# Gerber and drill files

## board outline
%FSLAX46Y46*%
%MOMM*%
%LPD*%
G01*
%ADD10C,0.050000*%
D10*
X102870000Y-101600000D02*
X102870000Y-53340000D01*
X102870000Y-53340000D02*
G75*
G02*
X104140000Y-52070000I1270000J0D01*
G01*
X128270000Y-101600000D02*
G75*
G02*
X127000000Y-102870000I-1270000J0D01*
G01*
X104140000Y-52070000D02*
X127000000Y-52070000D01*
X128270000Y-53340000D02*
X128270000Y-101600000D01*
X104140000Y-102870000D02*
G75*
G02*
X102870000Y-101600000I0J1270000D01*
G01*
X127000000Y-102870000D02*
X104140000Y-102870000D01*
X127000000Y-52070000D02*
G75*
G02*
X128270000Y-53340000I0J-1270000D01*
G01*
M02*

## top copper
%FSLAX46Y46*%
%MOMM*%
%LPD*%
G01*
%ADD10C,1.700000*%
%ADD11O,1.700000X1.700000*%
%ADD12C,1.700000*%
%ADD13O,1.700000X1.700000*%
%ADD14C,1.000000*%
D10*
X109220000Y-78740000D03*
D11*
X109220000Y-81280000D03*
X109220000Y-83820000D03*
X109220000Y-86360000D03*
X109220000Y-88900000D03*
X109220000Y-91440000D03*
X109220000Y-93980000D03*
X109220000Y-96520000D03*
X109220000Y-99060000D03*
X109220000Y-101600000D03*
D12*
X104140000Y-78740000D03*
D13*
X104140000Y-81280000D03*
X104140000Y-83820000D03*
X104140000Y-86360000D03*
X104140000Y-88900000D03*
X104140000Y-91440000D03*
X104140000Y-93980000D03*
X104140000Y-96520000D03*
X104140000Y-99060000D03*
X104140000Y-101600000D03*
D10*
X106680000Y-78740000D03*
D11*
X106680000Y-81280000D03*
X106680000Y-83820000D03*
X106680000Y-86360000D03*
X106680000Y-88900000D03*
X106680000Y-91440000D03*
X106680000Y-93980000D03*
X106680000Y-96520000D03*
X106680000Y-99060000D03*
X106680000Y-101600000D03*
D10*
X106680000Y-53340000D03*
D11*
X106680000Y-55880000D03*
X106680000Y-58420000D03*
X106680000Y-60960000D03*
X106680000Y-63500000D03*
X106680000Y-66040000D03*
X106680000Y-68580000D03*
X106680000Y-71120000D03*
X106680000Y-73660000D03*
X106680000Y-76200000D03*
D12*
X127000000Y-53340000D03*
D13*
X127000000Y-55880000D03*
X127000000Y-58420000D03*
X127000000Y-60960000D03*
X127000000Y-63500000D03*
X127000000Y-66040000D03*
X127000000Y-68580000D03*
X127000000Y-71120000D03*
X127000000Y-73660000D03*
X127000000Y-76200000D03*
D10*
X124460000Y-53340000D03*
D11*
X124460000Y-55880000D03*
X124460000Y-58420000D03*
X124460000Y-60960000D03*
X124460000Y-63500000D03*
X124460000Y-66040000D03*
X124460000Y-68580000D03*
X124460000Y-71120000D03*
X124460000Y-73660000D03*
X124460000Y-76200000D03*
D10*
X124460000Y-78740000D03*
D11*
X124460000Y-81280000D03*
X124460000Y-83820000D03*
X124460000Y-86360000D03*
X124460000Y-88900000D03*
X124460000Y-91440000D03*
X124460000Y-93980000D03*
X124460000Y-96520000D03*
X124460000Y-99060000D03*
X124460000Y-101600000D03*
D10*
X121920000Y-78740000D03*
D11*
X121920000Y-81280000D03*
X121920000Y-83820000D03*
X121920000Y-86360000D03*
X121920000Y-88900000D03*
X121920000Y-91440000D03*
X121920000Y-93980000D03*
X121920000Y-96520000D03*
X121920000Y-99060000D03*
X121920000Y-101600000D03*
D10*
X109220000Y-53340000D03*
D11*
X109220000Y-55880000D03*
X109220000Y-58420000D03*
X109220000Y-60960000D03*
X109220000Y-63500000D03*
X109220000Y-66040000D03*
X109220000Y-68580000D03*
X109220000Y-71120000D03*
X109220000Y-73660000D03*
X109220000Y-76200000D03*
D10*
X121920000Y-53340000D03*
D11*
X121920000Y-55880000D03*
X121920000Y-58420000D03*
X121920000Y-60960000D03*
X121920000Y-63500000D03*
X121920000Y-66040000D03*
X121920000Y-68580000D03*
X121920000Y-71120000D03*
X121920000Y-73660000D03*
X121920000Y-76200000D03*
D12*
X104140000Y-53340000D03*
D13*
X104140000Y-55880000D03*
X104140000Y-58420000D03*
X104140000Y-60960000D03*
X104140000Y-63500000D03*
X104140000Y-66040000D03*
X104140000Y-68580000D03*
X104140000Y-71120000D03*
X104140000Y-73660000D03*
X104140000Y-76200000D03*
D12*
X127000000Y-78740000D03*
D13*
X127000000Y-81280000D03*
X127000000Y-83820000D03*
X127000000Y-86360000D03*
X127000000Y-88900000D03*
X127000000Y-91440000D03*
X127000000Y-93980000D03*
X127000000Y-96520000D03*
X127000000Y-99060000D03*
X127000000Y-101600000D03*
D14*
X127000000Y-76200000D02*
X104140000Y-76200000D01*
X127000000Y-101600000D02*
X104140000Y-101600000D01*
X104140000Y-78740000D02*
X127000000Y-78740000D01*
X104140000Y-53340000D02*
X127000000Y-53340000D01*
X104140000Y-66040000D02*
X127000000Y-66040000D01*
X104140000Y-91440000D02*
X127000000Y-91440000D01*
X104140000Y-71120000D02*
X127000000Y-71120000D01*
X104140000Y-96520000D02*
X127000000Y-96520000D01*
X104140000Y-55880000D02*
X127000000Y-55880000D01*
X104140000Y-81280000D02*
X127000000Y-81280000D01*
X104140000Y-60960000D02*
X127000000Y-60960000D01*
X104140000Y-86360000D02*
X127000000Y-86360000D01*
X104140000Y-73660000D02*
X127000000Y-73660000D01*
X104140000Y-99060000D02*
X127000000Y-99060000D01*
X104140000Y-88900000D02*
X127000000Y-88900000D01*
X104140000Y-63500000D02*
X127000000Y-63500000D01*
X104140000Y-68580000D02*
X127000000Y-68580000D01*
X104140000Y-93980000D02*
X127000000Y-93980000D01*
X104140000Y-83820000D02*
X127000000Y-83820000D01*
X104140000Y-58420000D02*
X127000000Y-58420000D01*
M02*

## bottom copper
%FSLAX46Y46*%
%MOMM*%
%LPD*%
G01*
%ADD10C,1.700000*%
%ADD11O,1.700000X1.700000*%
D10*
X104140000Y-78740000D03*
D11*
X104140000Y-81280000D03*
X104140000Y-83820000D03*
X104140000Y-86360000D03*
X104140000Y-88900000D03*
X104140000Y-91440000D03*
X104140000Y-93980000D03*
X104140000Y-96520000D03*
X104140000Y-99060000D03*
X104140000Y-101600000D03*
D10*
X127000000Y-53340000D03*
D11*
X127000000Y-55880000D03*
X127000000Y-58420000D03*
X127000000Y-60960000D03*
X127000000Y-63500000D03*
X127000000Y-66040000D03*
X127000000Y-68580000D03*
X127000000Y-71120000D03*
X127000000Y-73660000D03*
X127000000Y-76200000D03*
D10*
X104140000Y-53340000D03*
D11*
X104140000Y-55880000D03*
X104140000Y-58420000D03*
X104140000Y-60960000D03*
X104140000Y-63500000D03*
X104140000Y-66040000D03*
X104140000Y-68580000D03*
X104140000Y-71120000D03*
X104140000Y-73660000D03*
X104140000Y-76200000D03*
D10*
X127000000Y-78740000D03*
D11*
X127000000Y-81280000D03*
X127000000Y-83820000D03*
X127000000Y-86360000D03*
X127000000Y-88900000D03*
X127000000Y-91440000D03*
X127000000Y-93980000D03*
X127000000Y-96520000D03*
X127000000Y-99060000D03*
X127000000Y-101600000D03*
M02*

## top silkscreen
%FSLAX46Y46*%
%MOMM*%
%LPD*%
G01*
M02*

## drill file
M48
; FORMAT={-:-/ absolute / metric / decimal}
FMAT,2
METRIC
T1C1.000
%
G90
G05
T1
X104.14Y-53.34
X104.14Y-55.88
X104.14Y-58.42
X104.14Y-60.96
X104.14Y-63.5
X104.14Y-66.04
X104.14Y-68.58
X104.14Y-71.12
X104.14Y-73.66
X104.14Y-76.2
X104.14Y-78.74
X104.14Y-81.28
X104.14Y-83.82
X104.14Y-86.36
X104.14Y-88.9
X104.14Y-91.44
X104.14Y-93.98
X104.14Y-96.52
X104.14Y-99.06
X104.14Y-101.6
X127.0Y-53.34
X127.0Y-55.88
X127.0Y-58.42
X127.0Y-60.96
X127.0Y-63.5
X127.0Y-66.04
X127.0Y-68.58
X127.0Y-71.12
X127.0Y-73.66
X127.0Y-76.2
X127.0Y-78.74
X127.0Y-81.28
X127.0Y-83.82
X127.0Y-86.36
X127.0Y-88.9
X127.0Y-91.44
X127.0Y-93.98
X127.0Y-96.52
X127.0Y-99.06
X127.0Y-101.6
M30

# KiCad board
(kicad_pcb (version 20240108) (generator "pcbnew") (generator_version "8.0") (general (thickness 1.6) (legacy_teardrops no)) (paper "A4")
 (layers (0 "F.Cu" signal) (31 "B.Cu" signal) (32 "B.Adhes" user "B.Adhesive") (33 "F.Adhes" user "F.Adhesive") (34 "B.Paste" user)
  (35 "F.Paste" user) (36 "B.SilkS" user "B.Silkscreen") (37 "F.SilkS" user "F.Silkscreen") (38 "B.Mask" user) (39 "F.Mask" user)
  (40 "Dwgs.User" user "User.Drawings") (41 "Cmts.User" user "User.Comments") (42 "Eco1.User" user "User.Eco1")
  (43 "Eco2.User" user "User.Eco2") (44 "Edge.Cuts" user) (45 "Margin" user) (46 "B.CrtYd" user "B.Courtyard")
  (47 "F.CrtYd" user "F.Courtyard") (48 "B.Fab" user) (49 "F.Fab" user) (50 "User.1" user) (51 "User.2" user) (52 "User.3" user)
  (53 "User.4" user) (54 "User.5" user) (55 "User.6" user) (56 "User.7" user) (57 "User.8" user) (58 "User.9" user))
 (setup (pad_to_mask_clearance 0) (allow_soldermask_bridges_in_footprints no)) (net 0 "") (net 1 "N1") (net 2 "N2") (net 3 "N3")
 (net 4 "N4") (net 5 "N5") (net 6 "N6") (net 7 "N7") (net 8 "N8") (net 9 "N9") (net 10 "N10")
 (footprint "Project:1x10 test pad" (layer "F.Cu") (at 109.22 90.065)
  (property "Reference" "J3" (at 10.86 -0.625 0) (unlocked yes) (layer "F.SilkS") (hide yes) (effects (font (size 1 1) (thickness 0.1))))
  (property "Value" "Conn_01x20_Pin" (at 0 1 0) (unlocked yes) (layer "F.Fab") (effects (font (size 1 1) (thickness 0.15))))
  (pad "1" smd circle (at 0 -11.325) (size 1.7 1.7) (layers "F.Cu" "F.Paste" "F.Mask") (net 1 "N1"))
  (pad "2" smd oval (at 0 -8.785) (size 1.7 1.7) (layers "F.Cu" "F.Paste" "F.Mask") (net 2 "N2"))
  (pad "3" smd oval (at 0 -6.245) (size 1.7 1.7) (layers "F.Cu" "F.Paste" "F.Mask") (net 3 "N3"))
  (pad "4" smd oval (at 0 -3.705) (size 1.7 1.7) (layers "F.Cu" "F.Paste" "F.Mask") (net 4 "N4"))
  (pad "5" smd oval (at 0 -1.165) (size 1.7 1.7) (layers "F.Cu" "F.Paste" "F.Mask") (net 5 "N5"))
  (pad "6" smd oval (at 0 1.375) (size 1.7 1.7) (layers "F.Cu" "F.Paste" "F.Mask") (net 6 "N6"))
  (pad "7" smd oval (at 0 3.915) (size 1.7 1.7) (layers "F.Cu" "F.Paste" "F.Mask") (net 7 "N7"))
  (pad "8" smd oval (at 0 6.455) (size 1.7 1.7) (layers "F.Cu" "F.Paste" "F.Mask") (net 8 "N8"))
  (pad "9" smd oval (at 0 8.995) (size 1.7 1.7) (layers "F.Cu" "F.Paste" "F.Mask") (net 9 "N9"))
  (pad "10" smd oval (at 0 11.535) (size 1.7 1.7) (layers "F.Cu" "F.Paste" "F.Mask") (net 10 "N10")))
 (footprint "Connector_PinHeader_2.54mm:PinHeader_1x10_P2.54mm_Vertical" (layer "F.Cu") (at 104.14 78.74)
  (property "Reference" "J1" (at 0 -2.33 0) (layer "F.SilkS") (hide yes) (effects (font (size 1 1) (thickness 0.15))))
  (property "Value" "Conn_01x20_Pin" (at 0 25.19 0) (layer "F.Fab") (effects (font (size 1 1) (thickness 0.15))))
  (pad "1" thru_hole circle (at 0 0) (size 1.7 1.7) (drill 1) (layers "*.Cu" "*.Mask") (remove_unused_layers no) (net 1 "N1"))
  (pad "2" thru_hole oval (at 0 2.54) (size 1.7 1.7) (drill 1) (layers "*.Cu" "*.Mask") (remove_unused_layers no) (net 2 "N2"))
  (pad "3" thru_hole oval (at 0 5.08) (size 1.7 1.7) (drill 1) (layers "*.Cu" "*.Mask") (remove_unused_layers no) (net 3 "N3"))
  (pad "4" thru_hole oval (at 0 7.62) (size 1.7 1.7) (drill 1) (layers "*.Cu" "*.Mask") (remove_unused_layers no) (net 4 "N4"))
  (pad "5" thru_hole oval (at 0 10.16) (size 1.7 1.7) (drill 1) (layers "*.Cu" "*.Mask") (remove_unused_layers no) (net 5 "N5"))
  (pad "6" thru_hole oval (at 0 12.7) (size 1.7 1.7) (drill 1) (layers "*.Cu" "*.Mask") (remove_unused_layers no) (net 6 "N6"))
  (pad "7" thru_hole oval (at 0 15.24) (size 1.7 1.7) (drill 1) (layers "*.Cu" "*.Mask") (remove_unused_layers no) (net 7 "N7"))
  (pad "8" thru_hole oval (at 0 17.78) (size 1.7 1.7) (drill 1) (layers "*.Cu" "*.Mask") (remove_unused_layers no) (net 8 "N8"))
  (pad "9" thru_hole oval (at 0 20.32) (size 1.7 1.7) (drill 1) (layers "*.Cu" "*.Mask") (remove_unused_layers no) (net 9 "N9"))
  (pad "10" thru_hole oval (at 0 22.86) (size 1.7 1.7) (drill 1) (layers "*.Cu" "*.Mask") (remove_unused_layers no) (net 10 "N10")))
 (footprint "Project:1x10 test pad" (layer "F.Cu") (at 106.68 90.065)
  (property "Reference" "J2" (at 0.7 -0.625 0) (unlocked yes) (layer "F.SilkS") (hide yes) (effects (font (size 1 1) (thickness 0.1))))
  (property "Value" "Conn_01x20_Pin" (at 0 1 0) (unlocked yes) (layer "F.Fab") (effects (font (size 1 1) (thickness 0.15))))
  (pad "1" smd circle (at 0 -11.325) (size 1.7 1.7) (layers "F.Cu" "F.Paste" "F.Mask") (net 1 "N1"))
  (pad "2" smd oval (at 0 -8.785) (size 1.7 1.7) (layers "F.Cu" "F.Paste" "F.Mask") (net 2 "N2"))
  (pad "3" smd oval (at 0 -6.245) (size 1.7 1.7) (layers "F.Cu" "F.Paste" "F.Mask") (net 3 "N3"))
  (pad "4" smd oval (at 0 -3.705) (size 1.7 1.7) (layers "F.Cu" "F.Paste" "F.Mask") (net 4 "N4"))
  (pad "5" smd oval (at 0 -1.165) (size 1.7 1.7) (layers "F.Cu" "F.Paste" "F.Mask") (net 5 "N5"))
  (pad "6" smd oval (at 0 1.375) (size 1.7 1.7) (layers "F.Cu" "F.Paste" "F.Mask") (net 6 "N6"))
  (pad "7" smd oval (at 0 3.915) (size 1.7 1.7) (layers "F.Cu" "F.Paste" "F.Mask") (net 7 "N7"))
  (pad "8" smd oval (at 0 6.455) (size 1.7 1.7) (layers "F.Cu" "F.Paste" "F.Mask") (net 8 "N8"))
  (pad "9" smd oval (at 0 8.995) (size 1.7 1.7) (layers "F.Cu" "F.Paste" "F.Mask") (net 9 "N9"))
  (pad "10" smd oval (at 0 11.535) (size 1.7 1.7) (layers "F.Cu" "F.Paste" "F.Mask") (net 10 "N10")))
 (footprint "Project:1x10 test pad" (layer "F.Cu") (at 106.68 64.665)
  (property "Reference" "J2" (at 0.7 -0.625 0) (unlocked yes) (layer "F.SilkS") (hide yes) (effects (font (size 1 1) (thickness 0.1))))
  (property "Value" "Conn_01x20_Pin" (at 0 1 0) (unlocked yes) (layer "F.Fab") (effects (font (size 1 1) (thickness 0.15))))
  (pad "1" smd circle (at 0 -11.325) (size 1.7 1.7) (layers "F.Cu" "F.Paste" "F.Mask") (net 1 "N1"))
  (pad "2" smd oval (at 0 -8.785) (size 1.7 1.7) (layers "F.Cu" "F.Paste" "F.Mask") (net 2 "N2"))
  (pad "3" smd oval (at 0 -6.245) (size 1.7 1.7) (layers "F.Cu" "F.Paste" "F.Mask") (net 3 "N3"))
  (pad "4" smd oval (at 0 -3.705) (size 1.7 1.7) (layers "F.Cu" "F.Paste" "F.Mask") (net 4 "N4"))
  (pad "5" smd oval (at 0 -1.165) (size 1.7 1.7) (layers "F.Cu" "F.Paste" "F.Mask") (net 5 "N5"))
  (pad "6" smd oval (at 0 1.375) (size 1.7 1.7) (layers "F.Cu" "F.Paste" "F.Mask") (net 6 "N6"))
  (pad "7" smd oval (at 0 3.915) (size 1.7 1.7) (layers "F.Cu" "F.Paste" "F.Mask") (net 7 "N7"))
  (pad "8" smd oval (at 0 6.455) (size 1.7 1.7) (layers "F.Cu" "F.Paste" "F.Mask") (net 8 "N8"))
  (pad "9" smd oval (at 0 8.995) (size 1.7 1.7) (layers "F.Cu" "F.Paste" "F.Mask") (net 9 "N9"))
  (pad "10" smd oval (at 0 11.535) (size 1.7 1.7) (layers "F.Cu" "F.Paste" "F.Mask") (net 10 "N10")))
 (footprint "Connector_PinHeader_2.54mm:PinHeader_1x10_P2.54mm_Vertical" (layer "F.Cu") (at 127 53.34)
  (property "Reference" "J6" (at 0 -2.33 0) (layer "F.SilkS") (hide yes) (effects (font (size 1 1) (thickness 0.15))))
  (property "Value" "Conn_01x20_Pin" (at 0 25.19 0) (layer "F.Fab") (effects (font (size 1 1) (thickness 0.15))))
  (pad "1" thru_hole circle (at 0 0) (size 1.7 1.7) (drill 1) (layers "*.Cu" "*.Mask") (remove_unused_layers no) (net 1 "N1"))
  (pad "2" thru_hole oval (at 0 2.54) (size 1.7 1.7) (drill 1) (layers "*.Cu" "*.Mask") (remove_unused_layers no) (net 2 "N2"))
  (pad "3" thru_hole oval (at 0 5.08) (size 1.7 1.7) (drill 1) (layers "*.Cu" "*.Mask") (remove_unused_layers no) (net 3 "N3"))
  (pad "4" thru_hole oval (at 0 7.62) (size 1.7 1.7) (drill 1) (layers "*.Cu" "*.Mask") (remove_unused_layers no) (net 4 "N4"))
  (pad "5" thru_hole oval (at 0 10.16) (size 1.7 1.7) (drill 1) (layers "*.Cu" "*.Mask") (remove_unused_layers no) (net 5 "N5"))
  (pad "6" thru_hole oval (at 0 12.7) (size 1.7 1.7) (drill 1) (layers "*.Cu" "*.Mask") (remove_unused_layers no) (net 6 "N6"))
  (pad "7" thru_hole oval (at 0 15.24) (size 1.7 1.7) (drill 1) (layers "*.Cu" "*.Mask") (remove_unused_layers no) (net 7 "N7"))
  (pad "8" thru_hole oval (at 0 17.78) (size 1.7 1.7) (drill 1) (layers "*.Cu" "*.Mask") (remove_unused_layers no) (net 8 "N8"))
  (pad "9" thru_hole oval (at 0 20.32) (size 1.7 1.7) (drill 1) (layers "*.Cu" "*.Mask") (remove_unused_layers no) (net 9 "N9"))
  (pad "10" thru_hole oval (at 0 22.86) (size 1.7 1.7) (drill 1) (layers "*.Cu" "*.Mask") (remove_unused_layers no) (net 10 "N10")))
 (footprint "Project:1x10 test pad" (layer "F.Cu") (at 124.46 64.665)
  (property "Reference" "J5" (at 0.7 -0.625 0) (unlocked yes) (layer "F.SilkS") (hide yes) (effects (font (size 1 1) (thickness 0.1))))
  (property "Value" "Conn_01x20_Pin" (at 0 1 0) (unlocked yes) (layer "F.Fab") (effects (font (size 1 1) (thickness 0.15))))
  (pad "1" smd circle (at 0 -11.325) (size 1.7 1.7) (layers "F.Cu" "F.Paste" "F.Mask") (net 1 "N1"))
  (pad "2" smd oval (at 0 -8.785) (size 1.7 1.7) (layers "F.Cu" "F.Paste" "F.Mask") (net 2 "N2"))
  (pad "3" smd oval (at 0 -6.245) (size 1.7 1.7) (layers "F.Cu" "F.Paste" "F.Mask") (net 3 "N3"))
  (pad "4" smd oval (at 0 -3.705) (size 1.7 1.7) (layers "F.Cu" "F.Paste" "F.Mask") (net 4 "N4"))
  (pad "5" smd oval (at 0 -1.165) (size 1.7 1.7) (layers "F.Cu" "F.Paste" "F.Mask") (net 5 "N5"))
  (pad "6" smd oval (at 0 1.375) (size 1.7 1.7) (layers "F.Cu" "F.Paste" "F.Mask") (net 6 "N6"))
  (pad "7" smd oval (at 0 3.915) (size 1.7 1.7) (layers "F.Cu" "F.Paste" "F.Mask") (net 7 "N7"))
  (pad "8" smd oval (at 0 6.455) (size 1.7 1.7) (layers "F.Cu" "F.Paste" "F.Mask") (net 8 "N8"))
  (pad "9" smd oval (at 0 8.995) (size 1.7 1.7) (layers "F.Cu" "F.Paste" "F.Mask") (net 9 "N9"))
  (pad "10" smd oval (at 0 11.535) (size 1.7 1.7) (layers "F.Cu" "F.Paste" "F.Mask") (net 10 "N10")))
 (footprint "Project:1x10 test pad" (layer "F.Cu") (at 124.46 90.065)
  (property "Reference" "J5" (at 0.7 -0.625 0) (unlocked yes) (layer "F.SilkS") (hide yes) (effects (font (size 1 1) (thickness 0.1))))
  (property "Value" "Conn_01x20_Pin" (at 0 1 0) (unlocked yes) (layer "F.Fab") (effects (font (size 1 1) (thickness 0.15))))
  (pad "1" smd circle (at 0 -11.325) (size 1.7 1.7) (layers "F.Cu" "F.Paste" "F.Mask") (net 1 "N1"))
  (pad "2" smd oval (at 0 -8.785) (size 1.7 1.7) (layers "F.Cu" "F.Paste" "F.Mask") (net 2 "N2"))
  (pad "3" smd oval (at 0 -6.245) (size 1.7 1.7) (layers "F.Cu" "F.Paste" "F.Mask") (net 3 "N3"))
  (pad "4" smd oval (at 0 -3.705) (size 1.7 1.7) (layers "F.Cu" "F.Paste" "F.Mask") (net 4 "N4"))
  (pad "5" smd oval (at 0 -1.165) (size 1.7 1.7) (layers "F.Cu" "F.Paste" "F.Mask") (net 5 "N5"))
  (pad "6" smd oval (at 0 1.375) (size 1.7 1.7) (layers "F.Cu" "F.Paste" "F.Mask") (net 6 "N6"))
  (pad "7" smd oval (at 0 3.915) (size 1.7 1.7) (layers "F.Cu" "F.Paste" "F.Mask") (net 7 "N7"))
  (pad "8" smd oval (at 0 6.455) (size 1.7 1.7) (layers "F.Cu" "F.Paste" "F.Mask") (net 8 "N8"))
  (pad "9" smd oval (at 0 8.995) (size 1.7 1.7) (layers "F.Cu" "F.Paste" "F.Mask") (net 9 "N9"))
  (pad "10" smd oval (at 0 11.535) (size 1.7 1.7) (layers "F.Cu" "F.Paste" "F.Mask") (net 10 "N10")))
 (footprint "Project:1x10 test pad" (layer "F.Cu") (at 121.92 90.065)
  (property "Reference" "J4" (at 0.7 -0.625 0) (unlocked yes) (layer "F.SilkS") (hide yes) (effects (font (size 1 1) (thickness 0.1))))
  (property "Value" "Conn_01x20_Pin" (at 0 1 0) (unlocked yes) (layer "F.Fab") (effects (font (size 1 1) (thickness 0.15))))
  (pad "1" smd circle (at 0 -11.325) (size 1.7 1.7) (layers "F.Cu" "F.Paste" "F.Mask") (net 1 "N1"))
  (pad "2" smd oval (at 0 -8.785) (size 1.7 1.7) (layers "F.Cu" "F.Paste" "F.Mask") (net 2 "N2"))
  (pad "3" smd oval (at 0 -6.245) (size 1.7 1.7) (layers "F.Cu" "F.Paste" "F.Mask") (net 3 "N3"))
  (pad "4" smd oval (at 0 -3.705) (size 1.7 1.7) (layers "F.Cu" "F.Paste" "F.Mask") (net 4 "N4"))
  (pad "5" smd oval (at 0 -1.165) (size 1.7 1.7) (layers "F.Cu" "F.Paste" "F.Mask") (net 5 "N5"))
  (pad "6" smd oval (at 0 1.375) (size 1.7 1.7) (layers "F.Cu" "F.Paste" "F.Mask") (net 6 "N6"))
  (pad "7" smd oval (at 0 3.915) (size 1.7 1.7) (layers "F.Cu" "F.Paste" "F.Mask") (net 7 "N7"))
  (pad "8" smd oval (at 0 6.455) (size 1.7 1.7) (layers "F.Cu" "F.Paste" "F.Mask") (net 8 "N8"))
  (pad "9" smd oval (at 0 8.995) (size 1.7 1.7) (layers "F.Cu" "F.Paste" "F.Mask") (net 9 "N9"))
  (pad "10" smd oval (at 0 11.535) (size 1.7 1.7) (layers "F.Cu" "F.Paste" "F.Mask") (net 10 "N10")))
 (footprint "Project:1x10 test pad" (layer "F.Cu") (at 109.22 64.665)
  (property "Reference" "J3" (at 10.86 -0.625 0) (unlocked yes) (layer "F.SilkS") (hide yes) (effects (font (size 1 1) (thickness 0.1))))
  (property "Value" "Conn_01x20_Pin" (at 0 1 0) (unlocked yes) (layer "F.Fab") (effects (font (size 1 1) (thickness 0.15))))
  (pad "1" smd circle (at 0 -11.325) (size 1.7 1.7) (layers "F.Cu" "F.Paste" "F.Mask") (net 1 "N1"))
  (pad "2" smd oval (at 0 -8.785) (size 1.7 1.7) (layers "F.Cu" "F.Paste" "F.Mask") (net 2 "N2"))
  (pad "3" smd oval (at 0 -6.245) (size 1.7 1.7) (layers "F.Cu" "F.Paste" "F.Mask") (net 3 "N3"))
  (pad "4" smd oval (at 0 -3.705) (size 1.7 1.7) (layers "F.Cu" "F.Paste" "F.Mask") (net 4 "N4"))
  (pad "5" smd oval (at 0 -1.165) (size 1.7 1.7) (layers "F.Cu" "F.Paste" "F.Mask") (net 5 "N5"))
  (pad "6" smd oval (at 0 1.375) (size 1.7 1.7) (layers "F.Cu" "F.Paste" "F.Mask") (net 6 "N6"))
  (pad "7" smd oval (at 0 3.915) (size 1.7 1.7) (layers "F.Cu" "F.Paste" "F.Mask") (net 7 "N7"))
  (pad "8" smd oval (at 0 6.455) (size 1.7 1.7) (layers "F.Cu" "F.Paste" "F.Mask") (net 8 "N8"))
  (pad "9" smd oval (at 0 8.995) (size 1.7 1.7) (layers "F.Cu" "F.Paste" "F.Mask") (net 9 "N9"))
  (pad "10" smd oval (at 0 11.535) (size 1.7 1.7) (layers "F.Cu" "F.Paste" "F.Mask") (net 10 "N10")))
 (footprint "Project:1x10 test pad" (layer "F.Cu") (at 121.92 64.665)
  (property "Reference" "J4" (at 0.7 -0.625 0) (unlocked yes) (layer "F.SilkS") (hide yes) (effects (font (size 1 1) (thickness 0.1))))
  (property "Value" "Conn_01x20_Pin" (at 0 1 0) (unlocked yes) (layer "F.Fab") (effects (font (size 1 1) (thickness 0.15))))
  (pad "1" smd circle (at 0 -11.325) (size 1.7 1.7) (layers "F.Cu" "F.Paste" "F.Mask") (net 1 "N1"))
  (pad "2" smd oval (at 0 -8.785) (size 1.7 1.7) (layers "F.Cu" "F.Paste" "F.Mask") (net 2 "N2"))
  (pad "3" smd oval (at 0 -6.245) (size 1.7 1.7) (layers "F.Cu" "F.Paste" "F.Mask") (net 3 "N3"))
  (pad "4" smd oval (at 0 -3.705) (size 1.7 1.7) (layers "F.Cu" "F.Paste" "F.Mask") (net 4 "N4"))
  (pad "5" smd oval (at 0 -1.165) (size 1.7 1.7) (layers "F.Cu" "F.Paste" "F.Mask") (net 5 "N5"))
  (pad "6" smd oval (at 0 1.375) (size 1.7 1.7) (layers "F.Cu" "F.Paste" "F.Mask") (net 6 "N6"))
  (pad "7" smd oval (at 0 3.915) (size 1.7 1.7) (layers "F.Cu" "F.Paste" "F.Mask") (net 7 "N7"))
  (pad "8" smd oval (at 0 6.455) (size 1.7 1.7) (layers "F.Cu" "F.Paste" "F.Mask") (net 8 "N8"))
  (pad "9" smd oval (at 0 8.995) (size 1.7 1.7) (layers "F.Cu" "F.Paste" "F.Mask") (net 9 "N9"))
  (pad "10" smd oval (at 0 11.535) (size 1.7 1.7) (layers "F.Cu" "F.Paste" "F.Mask") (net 10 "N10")))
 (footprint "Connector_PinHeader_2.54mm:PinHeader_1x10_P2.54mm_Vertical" (layer "F.Cu") (at 104.14 53.34)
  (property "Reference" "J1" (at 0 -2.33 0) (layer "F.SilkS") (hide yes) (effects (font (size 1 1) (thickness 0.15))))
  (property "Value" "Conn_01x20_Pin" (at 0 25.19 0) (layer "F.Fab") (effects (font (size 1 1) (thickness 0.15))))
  (pad "1" thru_hole circle (at 0 0) (size 1.7 1.7) (drill 1) (layers "*.Cu" "*.Mask") (remove_unused_layers no) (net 1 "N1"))
  (pad "2" thru_hole oval (at 0 2.54) (size 1.7 1.7) (drill 1) (layers "*.Cu" "*.Mask") (remove_unused_layers no) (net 2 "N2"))
  (pad "3" thru_hole oval (at 0 5.08) (size 1.7 1.7) (drill 1) (layers "*.Cu" "*.Mask") (remove_unused_layers no) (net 3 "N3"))
  (pad "4" thru_hole oval (at 0 7.62) (size 1.7 1.7) (drill 1) (layers "*.Cu" "*.Mask") (remove_unused_layers no) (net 4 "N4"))
  (pad "5" thru_hole oval (at 0 10.16) (size 1.7 1.7) (drill 1) (layers "*.Cu" "*.Mask") (remove_unused_layers no) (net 5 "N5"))
  (pad "6" thru_hole oval (at 0 12.7) (size 1.7 1.7) (drill 1) (layers "*.Cu" "*.Mask") (remove_unused_layers no) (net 6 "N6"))
  (pad "7" thru_hole oval (at 0 15.24) (size 1.7 1.7) (drill 1) (layers "*.Cu" "*.Mask") (remove_unused_layers no) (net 7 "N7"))
  (pad "8" thru_hole oval (at 0 17.78) (size 1.7 1.7) (drill 1) (layers "*.Cu" "*.Mask") (remove_unused_layers no) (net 8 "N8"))
  (pad "9" thru_hole oval (at 0 20.32) (size 1.7 1.7) (drill 1) (layers "*.Cu" "*.Mask") (remove_unused_layers no) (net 9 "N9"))
  (pad "10" thru_hole oval (at 0 22.86) (size 1.7 1.7) (drill 1) (layers "*.Cu" "*.Mask") (remove_unused_layers no) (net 10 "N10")))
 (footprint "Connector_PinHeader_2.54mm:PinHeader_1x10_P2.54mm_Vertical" (layer "F.Cu") (at 127 78.74)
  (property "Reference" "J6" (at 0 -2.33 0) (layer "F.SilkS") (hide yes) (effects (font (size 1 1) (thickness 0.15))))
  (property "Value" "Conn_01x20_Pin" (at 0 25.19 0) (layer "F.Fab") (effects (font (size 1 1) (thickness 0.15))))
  (pad "1" thru_hole circle (at 0 0) (size 1.7 1.7) (drill 1) (layers "*.Cu" "*.Mask") (remove_unused_layers no) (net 1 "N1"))
  (pad "2" thru_hole oval (at 0 2.54) (size 1.7 1.7) (drill 1) (layers "*.Cu" "*.Mask") (remove_unused_layers no) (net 2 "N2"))
  (pad "3" thru_hole oval (at 0 5.08) (size 1.7 1.7) (drill 1) (layers "*.Cu" "*.Mask") (remove_unused_layers no) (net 3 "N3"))
  (pad "4" thru_hole oval (at 0 7.62) (size 1.7 1.7) (drill 1) (layers "*.Cu" "*.Mask") (remove_unused_layers no) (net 4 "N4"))
  (pad "5" thru_hole oval (at 0 10.16) (size 1.7 1.7) (drill 1) (layers "*.Cu" "*.Mask") (remove_unused_layers no) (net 5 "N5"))
  (pad "6" thru_hole oval (at 0 12.7) (size 1.7 1.7) (drill 1) (layers "*.Cu" "*.Mask") (remove_unused_layers no) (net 6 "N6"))
  (pad "7" thru_hole oval (at 0 15.24) (size 1.7 1.7) (drill 1) (layers "*.Cu" "*.Mask") (remove_unused_layers no) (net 7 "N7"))
  (pad "8" thru_hole oval (at 0 17.78) (size 1.7 1.7) (drill 1) (layers "*.Cu" "*.Mask") (remove_unused_layers no) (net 8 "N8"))
  (pad "9" thru_hole oval (at 0 20.32) (size 1.7 1.7) (drill 1) (layers "*.Cu" "*.Mask") (remove_unused_layers no) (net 9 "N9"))
  (pad "10" thru_hole oval (at 0 22.86) (size 1.7 1.7) (drill 1) (layers "*.Cu" "*.Mask") (remove_unused_layers no) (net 10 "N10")))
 (gr_line (start 102.87 101.6) (end 102.87 53.34) (stroke (width 0.05) (type default)) (layer "Edge.Cuts"))
 (gr_arc (start 102.87 53.34) (mid 103.241974 52.441974) (end 104.14 52.07) (stroke (width 0.05) (type default)) (layer "Edge.Cuts"))
 (gr_arc (start 128.27 101.6) (mid 127.898026 102.498026) (end 127 102.87) (stroke (width 0.05) (type default)) (layer "Edge.Cuts"))
 (gr_line (start 104.14 52.07) (end 127 52.07) (stroke (width 0.05) (type default)) (layer "Edge.Cuts"))
 (gr_line (start 128.27 53.34) (end 128.27 101.6) (stroke (width 0.05) (type default)) (layer "Edge.Cuts"))
 (gr_arc (start 104.14 102.87) (mid 103.241974 102.498026) (end 102.87 101.6) (stroke (width 0.05) (type default)) (layer "Edge.Cuts"))
 (gr_line (start 127 102.87) (end 104.14 102.87) (stroke (width 0.05) (type default)) (layer "Edge.Cuts"))
 (gr_arc (start 127 52.07) (mid 127.898026 52.441974) (end 128.27 53.34) (stroke (width 0.05) (type default)) (layer "Edge.Cuts"))
 (segment (start 127 76.2) (end 104.14 76.2) (width 1) (layer "F.Cu") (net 10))
 (segment (start 127 101.6) (end 104.14 101.6) (width 1) (layer "F.Cu") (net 10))
 (segment (start 104.14 78.74) (end 127 78.74) (width 1) (layer "F.Cu") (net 1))
 (segment (start 104.14 53.34) (end 127 53.34) (width 1) (layer "F.Cu") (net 1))
 (segment (start 104.14 66.04) (end 127 66.04) (width 1) (layer "F.Cu") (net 6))
 (segment (start 104.14 91.44) (end 127 91.44) (width 1) (layer "F.Cu") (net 6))
 (segment (start 104.14 71.12) (end 127 71.12) (width 1) (layer "F.Cu") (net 8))
 (segment (start 104.14 96.52) (end 127 96.52) (width 1) (layer "F.Cu") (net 8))
 (segment (start 104.14 55.88) (end 127 55.88) (width 1) (layer "F.Cu") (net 2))
 (segment (start 104.14 81.28) (end 127 81.28) (width 1) (layer "F.Cu") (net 2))
 (segment (start 104.14 60.96) (end 127 60.96) (width 1) (layer "F.Cu") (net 4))
 (segment (start 104.14 86.36) (end 127 86.36) (width 1) (layer "F.Cu") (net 4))
 (segment (start 104.14 73.66) (end 127 73.66) (width 1) (layer "F.Cu") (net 9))
 (segment (start 104.14 99.06) (end 127 99.06) (width 1) (layer "F.Cu") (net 9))
 (segment (start 104.14 88.9) (end 127 88.9) (width 1) (layer "F.Cu") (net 5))
 (segment (start 104.14 63.5) (end 127 63.5) (width 1) (layer "F.Cu") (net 5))
 (segment (start 104.14 68.58) (end 127 68.58) (width 1) (layer "F.Cu") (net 7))
 (segment (start 104.14 93.98) (end 127 93.98) (width 1) (layer "F.Cu") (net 7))
 (segment (start 104.14 83.82) (end 127 83.82) (width 1) (layer "F.Cu") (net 3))
 (segment (start 104.14 58.42) (end 127 58.42) (width 1) (layer "F.Cu") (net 3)))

